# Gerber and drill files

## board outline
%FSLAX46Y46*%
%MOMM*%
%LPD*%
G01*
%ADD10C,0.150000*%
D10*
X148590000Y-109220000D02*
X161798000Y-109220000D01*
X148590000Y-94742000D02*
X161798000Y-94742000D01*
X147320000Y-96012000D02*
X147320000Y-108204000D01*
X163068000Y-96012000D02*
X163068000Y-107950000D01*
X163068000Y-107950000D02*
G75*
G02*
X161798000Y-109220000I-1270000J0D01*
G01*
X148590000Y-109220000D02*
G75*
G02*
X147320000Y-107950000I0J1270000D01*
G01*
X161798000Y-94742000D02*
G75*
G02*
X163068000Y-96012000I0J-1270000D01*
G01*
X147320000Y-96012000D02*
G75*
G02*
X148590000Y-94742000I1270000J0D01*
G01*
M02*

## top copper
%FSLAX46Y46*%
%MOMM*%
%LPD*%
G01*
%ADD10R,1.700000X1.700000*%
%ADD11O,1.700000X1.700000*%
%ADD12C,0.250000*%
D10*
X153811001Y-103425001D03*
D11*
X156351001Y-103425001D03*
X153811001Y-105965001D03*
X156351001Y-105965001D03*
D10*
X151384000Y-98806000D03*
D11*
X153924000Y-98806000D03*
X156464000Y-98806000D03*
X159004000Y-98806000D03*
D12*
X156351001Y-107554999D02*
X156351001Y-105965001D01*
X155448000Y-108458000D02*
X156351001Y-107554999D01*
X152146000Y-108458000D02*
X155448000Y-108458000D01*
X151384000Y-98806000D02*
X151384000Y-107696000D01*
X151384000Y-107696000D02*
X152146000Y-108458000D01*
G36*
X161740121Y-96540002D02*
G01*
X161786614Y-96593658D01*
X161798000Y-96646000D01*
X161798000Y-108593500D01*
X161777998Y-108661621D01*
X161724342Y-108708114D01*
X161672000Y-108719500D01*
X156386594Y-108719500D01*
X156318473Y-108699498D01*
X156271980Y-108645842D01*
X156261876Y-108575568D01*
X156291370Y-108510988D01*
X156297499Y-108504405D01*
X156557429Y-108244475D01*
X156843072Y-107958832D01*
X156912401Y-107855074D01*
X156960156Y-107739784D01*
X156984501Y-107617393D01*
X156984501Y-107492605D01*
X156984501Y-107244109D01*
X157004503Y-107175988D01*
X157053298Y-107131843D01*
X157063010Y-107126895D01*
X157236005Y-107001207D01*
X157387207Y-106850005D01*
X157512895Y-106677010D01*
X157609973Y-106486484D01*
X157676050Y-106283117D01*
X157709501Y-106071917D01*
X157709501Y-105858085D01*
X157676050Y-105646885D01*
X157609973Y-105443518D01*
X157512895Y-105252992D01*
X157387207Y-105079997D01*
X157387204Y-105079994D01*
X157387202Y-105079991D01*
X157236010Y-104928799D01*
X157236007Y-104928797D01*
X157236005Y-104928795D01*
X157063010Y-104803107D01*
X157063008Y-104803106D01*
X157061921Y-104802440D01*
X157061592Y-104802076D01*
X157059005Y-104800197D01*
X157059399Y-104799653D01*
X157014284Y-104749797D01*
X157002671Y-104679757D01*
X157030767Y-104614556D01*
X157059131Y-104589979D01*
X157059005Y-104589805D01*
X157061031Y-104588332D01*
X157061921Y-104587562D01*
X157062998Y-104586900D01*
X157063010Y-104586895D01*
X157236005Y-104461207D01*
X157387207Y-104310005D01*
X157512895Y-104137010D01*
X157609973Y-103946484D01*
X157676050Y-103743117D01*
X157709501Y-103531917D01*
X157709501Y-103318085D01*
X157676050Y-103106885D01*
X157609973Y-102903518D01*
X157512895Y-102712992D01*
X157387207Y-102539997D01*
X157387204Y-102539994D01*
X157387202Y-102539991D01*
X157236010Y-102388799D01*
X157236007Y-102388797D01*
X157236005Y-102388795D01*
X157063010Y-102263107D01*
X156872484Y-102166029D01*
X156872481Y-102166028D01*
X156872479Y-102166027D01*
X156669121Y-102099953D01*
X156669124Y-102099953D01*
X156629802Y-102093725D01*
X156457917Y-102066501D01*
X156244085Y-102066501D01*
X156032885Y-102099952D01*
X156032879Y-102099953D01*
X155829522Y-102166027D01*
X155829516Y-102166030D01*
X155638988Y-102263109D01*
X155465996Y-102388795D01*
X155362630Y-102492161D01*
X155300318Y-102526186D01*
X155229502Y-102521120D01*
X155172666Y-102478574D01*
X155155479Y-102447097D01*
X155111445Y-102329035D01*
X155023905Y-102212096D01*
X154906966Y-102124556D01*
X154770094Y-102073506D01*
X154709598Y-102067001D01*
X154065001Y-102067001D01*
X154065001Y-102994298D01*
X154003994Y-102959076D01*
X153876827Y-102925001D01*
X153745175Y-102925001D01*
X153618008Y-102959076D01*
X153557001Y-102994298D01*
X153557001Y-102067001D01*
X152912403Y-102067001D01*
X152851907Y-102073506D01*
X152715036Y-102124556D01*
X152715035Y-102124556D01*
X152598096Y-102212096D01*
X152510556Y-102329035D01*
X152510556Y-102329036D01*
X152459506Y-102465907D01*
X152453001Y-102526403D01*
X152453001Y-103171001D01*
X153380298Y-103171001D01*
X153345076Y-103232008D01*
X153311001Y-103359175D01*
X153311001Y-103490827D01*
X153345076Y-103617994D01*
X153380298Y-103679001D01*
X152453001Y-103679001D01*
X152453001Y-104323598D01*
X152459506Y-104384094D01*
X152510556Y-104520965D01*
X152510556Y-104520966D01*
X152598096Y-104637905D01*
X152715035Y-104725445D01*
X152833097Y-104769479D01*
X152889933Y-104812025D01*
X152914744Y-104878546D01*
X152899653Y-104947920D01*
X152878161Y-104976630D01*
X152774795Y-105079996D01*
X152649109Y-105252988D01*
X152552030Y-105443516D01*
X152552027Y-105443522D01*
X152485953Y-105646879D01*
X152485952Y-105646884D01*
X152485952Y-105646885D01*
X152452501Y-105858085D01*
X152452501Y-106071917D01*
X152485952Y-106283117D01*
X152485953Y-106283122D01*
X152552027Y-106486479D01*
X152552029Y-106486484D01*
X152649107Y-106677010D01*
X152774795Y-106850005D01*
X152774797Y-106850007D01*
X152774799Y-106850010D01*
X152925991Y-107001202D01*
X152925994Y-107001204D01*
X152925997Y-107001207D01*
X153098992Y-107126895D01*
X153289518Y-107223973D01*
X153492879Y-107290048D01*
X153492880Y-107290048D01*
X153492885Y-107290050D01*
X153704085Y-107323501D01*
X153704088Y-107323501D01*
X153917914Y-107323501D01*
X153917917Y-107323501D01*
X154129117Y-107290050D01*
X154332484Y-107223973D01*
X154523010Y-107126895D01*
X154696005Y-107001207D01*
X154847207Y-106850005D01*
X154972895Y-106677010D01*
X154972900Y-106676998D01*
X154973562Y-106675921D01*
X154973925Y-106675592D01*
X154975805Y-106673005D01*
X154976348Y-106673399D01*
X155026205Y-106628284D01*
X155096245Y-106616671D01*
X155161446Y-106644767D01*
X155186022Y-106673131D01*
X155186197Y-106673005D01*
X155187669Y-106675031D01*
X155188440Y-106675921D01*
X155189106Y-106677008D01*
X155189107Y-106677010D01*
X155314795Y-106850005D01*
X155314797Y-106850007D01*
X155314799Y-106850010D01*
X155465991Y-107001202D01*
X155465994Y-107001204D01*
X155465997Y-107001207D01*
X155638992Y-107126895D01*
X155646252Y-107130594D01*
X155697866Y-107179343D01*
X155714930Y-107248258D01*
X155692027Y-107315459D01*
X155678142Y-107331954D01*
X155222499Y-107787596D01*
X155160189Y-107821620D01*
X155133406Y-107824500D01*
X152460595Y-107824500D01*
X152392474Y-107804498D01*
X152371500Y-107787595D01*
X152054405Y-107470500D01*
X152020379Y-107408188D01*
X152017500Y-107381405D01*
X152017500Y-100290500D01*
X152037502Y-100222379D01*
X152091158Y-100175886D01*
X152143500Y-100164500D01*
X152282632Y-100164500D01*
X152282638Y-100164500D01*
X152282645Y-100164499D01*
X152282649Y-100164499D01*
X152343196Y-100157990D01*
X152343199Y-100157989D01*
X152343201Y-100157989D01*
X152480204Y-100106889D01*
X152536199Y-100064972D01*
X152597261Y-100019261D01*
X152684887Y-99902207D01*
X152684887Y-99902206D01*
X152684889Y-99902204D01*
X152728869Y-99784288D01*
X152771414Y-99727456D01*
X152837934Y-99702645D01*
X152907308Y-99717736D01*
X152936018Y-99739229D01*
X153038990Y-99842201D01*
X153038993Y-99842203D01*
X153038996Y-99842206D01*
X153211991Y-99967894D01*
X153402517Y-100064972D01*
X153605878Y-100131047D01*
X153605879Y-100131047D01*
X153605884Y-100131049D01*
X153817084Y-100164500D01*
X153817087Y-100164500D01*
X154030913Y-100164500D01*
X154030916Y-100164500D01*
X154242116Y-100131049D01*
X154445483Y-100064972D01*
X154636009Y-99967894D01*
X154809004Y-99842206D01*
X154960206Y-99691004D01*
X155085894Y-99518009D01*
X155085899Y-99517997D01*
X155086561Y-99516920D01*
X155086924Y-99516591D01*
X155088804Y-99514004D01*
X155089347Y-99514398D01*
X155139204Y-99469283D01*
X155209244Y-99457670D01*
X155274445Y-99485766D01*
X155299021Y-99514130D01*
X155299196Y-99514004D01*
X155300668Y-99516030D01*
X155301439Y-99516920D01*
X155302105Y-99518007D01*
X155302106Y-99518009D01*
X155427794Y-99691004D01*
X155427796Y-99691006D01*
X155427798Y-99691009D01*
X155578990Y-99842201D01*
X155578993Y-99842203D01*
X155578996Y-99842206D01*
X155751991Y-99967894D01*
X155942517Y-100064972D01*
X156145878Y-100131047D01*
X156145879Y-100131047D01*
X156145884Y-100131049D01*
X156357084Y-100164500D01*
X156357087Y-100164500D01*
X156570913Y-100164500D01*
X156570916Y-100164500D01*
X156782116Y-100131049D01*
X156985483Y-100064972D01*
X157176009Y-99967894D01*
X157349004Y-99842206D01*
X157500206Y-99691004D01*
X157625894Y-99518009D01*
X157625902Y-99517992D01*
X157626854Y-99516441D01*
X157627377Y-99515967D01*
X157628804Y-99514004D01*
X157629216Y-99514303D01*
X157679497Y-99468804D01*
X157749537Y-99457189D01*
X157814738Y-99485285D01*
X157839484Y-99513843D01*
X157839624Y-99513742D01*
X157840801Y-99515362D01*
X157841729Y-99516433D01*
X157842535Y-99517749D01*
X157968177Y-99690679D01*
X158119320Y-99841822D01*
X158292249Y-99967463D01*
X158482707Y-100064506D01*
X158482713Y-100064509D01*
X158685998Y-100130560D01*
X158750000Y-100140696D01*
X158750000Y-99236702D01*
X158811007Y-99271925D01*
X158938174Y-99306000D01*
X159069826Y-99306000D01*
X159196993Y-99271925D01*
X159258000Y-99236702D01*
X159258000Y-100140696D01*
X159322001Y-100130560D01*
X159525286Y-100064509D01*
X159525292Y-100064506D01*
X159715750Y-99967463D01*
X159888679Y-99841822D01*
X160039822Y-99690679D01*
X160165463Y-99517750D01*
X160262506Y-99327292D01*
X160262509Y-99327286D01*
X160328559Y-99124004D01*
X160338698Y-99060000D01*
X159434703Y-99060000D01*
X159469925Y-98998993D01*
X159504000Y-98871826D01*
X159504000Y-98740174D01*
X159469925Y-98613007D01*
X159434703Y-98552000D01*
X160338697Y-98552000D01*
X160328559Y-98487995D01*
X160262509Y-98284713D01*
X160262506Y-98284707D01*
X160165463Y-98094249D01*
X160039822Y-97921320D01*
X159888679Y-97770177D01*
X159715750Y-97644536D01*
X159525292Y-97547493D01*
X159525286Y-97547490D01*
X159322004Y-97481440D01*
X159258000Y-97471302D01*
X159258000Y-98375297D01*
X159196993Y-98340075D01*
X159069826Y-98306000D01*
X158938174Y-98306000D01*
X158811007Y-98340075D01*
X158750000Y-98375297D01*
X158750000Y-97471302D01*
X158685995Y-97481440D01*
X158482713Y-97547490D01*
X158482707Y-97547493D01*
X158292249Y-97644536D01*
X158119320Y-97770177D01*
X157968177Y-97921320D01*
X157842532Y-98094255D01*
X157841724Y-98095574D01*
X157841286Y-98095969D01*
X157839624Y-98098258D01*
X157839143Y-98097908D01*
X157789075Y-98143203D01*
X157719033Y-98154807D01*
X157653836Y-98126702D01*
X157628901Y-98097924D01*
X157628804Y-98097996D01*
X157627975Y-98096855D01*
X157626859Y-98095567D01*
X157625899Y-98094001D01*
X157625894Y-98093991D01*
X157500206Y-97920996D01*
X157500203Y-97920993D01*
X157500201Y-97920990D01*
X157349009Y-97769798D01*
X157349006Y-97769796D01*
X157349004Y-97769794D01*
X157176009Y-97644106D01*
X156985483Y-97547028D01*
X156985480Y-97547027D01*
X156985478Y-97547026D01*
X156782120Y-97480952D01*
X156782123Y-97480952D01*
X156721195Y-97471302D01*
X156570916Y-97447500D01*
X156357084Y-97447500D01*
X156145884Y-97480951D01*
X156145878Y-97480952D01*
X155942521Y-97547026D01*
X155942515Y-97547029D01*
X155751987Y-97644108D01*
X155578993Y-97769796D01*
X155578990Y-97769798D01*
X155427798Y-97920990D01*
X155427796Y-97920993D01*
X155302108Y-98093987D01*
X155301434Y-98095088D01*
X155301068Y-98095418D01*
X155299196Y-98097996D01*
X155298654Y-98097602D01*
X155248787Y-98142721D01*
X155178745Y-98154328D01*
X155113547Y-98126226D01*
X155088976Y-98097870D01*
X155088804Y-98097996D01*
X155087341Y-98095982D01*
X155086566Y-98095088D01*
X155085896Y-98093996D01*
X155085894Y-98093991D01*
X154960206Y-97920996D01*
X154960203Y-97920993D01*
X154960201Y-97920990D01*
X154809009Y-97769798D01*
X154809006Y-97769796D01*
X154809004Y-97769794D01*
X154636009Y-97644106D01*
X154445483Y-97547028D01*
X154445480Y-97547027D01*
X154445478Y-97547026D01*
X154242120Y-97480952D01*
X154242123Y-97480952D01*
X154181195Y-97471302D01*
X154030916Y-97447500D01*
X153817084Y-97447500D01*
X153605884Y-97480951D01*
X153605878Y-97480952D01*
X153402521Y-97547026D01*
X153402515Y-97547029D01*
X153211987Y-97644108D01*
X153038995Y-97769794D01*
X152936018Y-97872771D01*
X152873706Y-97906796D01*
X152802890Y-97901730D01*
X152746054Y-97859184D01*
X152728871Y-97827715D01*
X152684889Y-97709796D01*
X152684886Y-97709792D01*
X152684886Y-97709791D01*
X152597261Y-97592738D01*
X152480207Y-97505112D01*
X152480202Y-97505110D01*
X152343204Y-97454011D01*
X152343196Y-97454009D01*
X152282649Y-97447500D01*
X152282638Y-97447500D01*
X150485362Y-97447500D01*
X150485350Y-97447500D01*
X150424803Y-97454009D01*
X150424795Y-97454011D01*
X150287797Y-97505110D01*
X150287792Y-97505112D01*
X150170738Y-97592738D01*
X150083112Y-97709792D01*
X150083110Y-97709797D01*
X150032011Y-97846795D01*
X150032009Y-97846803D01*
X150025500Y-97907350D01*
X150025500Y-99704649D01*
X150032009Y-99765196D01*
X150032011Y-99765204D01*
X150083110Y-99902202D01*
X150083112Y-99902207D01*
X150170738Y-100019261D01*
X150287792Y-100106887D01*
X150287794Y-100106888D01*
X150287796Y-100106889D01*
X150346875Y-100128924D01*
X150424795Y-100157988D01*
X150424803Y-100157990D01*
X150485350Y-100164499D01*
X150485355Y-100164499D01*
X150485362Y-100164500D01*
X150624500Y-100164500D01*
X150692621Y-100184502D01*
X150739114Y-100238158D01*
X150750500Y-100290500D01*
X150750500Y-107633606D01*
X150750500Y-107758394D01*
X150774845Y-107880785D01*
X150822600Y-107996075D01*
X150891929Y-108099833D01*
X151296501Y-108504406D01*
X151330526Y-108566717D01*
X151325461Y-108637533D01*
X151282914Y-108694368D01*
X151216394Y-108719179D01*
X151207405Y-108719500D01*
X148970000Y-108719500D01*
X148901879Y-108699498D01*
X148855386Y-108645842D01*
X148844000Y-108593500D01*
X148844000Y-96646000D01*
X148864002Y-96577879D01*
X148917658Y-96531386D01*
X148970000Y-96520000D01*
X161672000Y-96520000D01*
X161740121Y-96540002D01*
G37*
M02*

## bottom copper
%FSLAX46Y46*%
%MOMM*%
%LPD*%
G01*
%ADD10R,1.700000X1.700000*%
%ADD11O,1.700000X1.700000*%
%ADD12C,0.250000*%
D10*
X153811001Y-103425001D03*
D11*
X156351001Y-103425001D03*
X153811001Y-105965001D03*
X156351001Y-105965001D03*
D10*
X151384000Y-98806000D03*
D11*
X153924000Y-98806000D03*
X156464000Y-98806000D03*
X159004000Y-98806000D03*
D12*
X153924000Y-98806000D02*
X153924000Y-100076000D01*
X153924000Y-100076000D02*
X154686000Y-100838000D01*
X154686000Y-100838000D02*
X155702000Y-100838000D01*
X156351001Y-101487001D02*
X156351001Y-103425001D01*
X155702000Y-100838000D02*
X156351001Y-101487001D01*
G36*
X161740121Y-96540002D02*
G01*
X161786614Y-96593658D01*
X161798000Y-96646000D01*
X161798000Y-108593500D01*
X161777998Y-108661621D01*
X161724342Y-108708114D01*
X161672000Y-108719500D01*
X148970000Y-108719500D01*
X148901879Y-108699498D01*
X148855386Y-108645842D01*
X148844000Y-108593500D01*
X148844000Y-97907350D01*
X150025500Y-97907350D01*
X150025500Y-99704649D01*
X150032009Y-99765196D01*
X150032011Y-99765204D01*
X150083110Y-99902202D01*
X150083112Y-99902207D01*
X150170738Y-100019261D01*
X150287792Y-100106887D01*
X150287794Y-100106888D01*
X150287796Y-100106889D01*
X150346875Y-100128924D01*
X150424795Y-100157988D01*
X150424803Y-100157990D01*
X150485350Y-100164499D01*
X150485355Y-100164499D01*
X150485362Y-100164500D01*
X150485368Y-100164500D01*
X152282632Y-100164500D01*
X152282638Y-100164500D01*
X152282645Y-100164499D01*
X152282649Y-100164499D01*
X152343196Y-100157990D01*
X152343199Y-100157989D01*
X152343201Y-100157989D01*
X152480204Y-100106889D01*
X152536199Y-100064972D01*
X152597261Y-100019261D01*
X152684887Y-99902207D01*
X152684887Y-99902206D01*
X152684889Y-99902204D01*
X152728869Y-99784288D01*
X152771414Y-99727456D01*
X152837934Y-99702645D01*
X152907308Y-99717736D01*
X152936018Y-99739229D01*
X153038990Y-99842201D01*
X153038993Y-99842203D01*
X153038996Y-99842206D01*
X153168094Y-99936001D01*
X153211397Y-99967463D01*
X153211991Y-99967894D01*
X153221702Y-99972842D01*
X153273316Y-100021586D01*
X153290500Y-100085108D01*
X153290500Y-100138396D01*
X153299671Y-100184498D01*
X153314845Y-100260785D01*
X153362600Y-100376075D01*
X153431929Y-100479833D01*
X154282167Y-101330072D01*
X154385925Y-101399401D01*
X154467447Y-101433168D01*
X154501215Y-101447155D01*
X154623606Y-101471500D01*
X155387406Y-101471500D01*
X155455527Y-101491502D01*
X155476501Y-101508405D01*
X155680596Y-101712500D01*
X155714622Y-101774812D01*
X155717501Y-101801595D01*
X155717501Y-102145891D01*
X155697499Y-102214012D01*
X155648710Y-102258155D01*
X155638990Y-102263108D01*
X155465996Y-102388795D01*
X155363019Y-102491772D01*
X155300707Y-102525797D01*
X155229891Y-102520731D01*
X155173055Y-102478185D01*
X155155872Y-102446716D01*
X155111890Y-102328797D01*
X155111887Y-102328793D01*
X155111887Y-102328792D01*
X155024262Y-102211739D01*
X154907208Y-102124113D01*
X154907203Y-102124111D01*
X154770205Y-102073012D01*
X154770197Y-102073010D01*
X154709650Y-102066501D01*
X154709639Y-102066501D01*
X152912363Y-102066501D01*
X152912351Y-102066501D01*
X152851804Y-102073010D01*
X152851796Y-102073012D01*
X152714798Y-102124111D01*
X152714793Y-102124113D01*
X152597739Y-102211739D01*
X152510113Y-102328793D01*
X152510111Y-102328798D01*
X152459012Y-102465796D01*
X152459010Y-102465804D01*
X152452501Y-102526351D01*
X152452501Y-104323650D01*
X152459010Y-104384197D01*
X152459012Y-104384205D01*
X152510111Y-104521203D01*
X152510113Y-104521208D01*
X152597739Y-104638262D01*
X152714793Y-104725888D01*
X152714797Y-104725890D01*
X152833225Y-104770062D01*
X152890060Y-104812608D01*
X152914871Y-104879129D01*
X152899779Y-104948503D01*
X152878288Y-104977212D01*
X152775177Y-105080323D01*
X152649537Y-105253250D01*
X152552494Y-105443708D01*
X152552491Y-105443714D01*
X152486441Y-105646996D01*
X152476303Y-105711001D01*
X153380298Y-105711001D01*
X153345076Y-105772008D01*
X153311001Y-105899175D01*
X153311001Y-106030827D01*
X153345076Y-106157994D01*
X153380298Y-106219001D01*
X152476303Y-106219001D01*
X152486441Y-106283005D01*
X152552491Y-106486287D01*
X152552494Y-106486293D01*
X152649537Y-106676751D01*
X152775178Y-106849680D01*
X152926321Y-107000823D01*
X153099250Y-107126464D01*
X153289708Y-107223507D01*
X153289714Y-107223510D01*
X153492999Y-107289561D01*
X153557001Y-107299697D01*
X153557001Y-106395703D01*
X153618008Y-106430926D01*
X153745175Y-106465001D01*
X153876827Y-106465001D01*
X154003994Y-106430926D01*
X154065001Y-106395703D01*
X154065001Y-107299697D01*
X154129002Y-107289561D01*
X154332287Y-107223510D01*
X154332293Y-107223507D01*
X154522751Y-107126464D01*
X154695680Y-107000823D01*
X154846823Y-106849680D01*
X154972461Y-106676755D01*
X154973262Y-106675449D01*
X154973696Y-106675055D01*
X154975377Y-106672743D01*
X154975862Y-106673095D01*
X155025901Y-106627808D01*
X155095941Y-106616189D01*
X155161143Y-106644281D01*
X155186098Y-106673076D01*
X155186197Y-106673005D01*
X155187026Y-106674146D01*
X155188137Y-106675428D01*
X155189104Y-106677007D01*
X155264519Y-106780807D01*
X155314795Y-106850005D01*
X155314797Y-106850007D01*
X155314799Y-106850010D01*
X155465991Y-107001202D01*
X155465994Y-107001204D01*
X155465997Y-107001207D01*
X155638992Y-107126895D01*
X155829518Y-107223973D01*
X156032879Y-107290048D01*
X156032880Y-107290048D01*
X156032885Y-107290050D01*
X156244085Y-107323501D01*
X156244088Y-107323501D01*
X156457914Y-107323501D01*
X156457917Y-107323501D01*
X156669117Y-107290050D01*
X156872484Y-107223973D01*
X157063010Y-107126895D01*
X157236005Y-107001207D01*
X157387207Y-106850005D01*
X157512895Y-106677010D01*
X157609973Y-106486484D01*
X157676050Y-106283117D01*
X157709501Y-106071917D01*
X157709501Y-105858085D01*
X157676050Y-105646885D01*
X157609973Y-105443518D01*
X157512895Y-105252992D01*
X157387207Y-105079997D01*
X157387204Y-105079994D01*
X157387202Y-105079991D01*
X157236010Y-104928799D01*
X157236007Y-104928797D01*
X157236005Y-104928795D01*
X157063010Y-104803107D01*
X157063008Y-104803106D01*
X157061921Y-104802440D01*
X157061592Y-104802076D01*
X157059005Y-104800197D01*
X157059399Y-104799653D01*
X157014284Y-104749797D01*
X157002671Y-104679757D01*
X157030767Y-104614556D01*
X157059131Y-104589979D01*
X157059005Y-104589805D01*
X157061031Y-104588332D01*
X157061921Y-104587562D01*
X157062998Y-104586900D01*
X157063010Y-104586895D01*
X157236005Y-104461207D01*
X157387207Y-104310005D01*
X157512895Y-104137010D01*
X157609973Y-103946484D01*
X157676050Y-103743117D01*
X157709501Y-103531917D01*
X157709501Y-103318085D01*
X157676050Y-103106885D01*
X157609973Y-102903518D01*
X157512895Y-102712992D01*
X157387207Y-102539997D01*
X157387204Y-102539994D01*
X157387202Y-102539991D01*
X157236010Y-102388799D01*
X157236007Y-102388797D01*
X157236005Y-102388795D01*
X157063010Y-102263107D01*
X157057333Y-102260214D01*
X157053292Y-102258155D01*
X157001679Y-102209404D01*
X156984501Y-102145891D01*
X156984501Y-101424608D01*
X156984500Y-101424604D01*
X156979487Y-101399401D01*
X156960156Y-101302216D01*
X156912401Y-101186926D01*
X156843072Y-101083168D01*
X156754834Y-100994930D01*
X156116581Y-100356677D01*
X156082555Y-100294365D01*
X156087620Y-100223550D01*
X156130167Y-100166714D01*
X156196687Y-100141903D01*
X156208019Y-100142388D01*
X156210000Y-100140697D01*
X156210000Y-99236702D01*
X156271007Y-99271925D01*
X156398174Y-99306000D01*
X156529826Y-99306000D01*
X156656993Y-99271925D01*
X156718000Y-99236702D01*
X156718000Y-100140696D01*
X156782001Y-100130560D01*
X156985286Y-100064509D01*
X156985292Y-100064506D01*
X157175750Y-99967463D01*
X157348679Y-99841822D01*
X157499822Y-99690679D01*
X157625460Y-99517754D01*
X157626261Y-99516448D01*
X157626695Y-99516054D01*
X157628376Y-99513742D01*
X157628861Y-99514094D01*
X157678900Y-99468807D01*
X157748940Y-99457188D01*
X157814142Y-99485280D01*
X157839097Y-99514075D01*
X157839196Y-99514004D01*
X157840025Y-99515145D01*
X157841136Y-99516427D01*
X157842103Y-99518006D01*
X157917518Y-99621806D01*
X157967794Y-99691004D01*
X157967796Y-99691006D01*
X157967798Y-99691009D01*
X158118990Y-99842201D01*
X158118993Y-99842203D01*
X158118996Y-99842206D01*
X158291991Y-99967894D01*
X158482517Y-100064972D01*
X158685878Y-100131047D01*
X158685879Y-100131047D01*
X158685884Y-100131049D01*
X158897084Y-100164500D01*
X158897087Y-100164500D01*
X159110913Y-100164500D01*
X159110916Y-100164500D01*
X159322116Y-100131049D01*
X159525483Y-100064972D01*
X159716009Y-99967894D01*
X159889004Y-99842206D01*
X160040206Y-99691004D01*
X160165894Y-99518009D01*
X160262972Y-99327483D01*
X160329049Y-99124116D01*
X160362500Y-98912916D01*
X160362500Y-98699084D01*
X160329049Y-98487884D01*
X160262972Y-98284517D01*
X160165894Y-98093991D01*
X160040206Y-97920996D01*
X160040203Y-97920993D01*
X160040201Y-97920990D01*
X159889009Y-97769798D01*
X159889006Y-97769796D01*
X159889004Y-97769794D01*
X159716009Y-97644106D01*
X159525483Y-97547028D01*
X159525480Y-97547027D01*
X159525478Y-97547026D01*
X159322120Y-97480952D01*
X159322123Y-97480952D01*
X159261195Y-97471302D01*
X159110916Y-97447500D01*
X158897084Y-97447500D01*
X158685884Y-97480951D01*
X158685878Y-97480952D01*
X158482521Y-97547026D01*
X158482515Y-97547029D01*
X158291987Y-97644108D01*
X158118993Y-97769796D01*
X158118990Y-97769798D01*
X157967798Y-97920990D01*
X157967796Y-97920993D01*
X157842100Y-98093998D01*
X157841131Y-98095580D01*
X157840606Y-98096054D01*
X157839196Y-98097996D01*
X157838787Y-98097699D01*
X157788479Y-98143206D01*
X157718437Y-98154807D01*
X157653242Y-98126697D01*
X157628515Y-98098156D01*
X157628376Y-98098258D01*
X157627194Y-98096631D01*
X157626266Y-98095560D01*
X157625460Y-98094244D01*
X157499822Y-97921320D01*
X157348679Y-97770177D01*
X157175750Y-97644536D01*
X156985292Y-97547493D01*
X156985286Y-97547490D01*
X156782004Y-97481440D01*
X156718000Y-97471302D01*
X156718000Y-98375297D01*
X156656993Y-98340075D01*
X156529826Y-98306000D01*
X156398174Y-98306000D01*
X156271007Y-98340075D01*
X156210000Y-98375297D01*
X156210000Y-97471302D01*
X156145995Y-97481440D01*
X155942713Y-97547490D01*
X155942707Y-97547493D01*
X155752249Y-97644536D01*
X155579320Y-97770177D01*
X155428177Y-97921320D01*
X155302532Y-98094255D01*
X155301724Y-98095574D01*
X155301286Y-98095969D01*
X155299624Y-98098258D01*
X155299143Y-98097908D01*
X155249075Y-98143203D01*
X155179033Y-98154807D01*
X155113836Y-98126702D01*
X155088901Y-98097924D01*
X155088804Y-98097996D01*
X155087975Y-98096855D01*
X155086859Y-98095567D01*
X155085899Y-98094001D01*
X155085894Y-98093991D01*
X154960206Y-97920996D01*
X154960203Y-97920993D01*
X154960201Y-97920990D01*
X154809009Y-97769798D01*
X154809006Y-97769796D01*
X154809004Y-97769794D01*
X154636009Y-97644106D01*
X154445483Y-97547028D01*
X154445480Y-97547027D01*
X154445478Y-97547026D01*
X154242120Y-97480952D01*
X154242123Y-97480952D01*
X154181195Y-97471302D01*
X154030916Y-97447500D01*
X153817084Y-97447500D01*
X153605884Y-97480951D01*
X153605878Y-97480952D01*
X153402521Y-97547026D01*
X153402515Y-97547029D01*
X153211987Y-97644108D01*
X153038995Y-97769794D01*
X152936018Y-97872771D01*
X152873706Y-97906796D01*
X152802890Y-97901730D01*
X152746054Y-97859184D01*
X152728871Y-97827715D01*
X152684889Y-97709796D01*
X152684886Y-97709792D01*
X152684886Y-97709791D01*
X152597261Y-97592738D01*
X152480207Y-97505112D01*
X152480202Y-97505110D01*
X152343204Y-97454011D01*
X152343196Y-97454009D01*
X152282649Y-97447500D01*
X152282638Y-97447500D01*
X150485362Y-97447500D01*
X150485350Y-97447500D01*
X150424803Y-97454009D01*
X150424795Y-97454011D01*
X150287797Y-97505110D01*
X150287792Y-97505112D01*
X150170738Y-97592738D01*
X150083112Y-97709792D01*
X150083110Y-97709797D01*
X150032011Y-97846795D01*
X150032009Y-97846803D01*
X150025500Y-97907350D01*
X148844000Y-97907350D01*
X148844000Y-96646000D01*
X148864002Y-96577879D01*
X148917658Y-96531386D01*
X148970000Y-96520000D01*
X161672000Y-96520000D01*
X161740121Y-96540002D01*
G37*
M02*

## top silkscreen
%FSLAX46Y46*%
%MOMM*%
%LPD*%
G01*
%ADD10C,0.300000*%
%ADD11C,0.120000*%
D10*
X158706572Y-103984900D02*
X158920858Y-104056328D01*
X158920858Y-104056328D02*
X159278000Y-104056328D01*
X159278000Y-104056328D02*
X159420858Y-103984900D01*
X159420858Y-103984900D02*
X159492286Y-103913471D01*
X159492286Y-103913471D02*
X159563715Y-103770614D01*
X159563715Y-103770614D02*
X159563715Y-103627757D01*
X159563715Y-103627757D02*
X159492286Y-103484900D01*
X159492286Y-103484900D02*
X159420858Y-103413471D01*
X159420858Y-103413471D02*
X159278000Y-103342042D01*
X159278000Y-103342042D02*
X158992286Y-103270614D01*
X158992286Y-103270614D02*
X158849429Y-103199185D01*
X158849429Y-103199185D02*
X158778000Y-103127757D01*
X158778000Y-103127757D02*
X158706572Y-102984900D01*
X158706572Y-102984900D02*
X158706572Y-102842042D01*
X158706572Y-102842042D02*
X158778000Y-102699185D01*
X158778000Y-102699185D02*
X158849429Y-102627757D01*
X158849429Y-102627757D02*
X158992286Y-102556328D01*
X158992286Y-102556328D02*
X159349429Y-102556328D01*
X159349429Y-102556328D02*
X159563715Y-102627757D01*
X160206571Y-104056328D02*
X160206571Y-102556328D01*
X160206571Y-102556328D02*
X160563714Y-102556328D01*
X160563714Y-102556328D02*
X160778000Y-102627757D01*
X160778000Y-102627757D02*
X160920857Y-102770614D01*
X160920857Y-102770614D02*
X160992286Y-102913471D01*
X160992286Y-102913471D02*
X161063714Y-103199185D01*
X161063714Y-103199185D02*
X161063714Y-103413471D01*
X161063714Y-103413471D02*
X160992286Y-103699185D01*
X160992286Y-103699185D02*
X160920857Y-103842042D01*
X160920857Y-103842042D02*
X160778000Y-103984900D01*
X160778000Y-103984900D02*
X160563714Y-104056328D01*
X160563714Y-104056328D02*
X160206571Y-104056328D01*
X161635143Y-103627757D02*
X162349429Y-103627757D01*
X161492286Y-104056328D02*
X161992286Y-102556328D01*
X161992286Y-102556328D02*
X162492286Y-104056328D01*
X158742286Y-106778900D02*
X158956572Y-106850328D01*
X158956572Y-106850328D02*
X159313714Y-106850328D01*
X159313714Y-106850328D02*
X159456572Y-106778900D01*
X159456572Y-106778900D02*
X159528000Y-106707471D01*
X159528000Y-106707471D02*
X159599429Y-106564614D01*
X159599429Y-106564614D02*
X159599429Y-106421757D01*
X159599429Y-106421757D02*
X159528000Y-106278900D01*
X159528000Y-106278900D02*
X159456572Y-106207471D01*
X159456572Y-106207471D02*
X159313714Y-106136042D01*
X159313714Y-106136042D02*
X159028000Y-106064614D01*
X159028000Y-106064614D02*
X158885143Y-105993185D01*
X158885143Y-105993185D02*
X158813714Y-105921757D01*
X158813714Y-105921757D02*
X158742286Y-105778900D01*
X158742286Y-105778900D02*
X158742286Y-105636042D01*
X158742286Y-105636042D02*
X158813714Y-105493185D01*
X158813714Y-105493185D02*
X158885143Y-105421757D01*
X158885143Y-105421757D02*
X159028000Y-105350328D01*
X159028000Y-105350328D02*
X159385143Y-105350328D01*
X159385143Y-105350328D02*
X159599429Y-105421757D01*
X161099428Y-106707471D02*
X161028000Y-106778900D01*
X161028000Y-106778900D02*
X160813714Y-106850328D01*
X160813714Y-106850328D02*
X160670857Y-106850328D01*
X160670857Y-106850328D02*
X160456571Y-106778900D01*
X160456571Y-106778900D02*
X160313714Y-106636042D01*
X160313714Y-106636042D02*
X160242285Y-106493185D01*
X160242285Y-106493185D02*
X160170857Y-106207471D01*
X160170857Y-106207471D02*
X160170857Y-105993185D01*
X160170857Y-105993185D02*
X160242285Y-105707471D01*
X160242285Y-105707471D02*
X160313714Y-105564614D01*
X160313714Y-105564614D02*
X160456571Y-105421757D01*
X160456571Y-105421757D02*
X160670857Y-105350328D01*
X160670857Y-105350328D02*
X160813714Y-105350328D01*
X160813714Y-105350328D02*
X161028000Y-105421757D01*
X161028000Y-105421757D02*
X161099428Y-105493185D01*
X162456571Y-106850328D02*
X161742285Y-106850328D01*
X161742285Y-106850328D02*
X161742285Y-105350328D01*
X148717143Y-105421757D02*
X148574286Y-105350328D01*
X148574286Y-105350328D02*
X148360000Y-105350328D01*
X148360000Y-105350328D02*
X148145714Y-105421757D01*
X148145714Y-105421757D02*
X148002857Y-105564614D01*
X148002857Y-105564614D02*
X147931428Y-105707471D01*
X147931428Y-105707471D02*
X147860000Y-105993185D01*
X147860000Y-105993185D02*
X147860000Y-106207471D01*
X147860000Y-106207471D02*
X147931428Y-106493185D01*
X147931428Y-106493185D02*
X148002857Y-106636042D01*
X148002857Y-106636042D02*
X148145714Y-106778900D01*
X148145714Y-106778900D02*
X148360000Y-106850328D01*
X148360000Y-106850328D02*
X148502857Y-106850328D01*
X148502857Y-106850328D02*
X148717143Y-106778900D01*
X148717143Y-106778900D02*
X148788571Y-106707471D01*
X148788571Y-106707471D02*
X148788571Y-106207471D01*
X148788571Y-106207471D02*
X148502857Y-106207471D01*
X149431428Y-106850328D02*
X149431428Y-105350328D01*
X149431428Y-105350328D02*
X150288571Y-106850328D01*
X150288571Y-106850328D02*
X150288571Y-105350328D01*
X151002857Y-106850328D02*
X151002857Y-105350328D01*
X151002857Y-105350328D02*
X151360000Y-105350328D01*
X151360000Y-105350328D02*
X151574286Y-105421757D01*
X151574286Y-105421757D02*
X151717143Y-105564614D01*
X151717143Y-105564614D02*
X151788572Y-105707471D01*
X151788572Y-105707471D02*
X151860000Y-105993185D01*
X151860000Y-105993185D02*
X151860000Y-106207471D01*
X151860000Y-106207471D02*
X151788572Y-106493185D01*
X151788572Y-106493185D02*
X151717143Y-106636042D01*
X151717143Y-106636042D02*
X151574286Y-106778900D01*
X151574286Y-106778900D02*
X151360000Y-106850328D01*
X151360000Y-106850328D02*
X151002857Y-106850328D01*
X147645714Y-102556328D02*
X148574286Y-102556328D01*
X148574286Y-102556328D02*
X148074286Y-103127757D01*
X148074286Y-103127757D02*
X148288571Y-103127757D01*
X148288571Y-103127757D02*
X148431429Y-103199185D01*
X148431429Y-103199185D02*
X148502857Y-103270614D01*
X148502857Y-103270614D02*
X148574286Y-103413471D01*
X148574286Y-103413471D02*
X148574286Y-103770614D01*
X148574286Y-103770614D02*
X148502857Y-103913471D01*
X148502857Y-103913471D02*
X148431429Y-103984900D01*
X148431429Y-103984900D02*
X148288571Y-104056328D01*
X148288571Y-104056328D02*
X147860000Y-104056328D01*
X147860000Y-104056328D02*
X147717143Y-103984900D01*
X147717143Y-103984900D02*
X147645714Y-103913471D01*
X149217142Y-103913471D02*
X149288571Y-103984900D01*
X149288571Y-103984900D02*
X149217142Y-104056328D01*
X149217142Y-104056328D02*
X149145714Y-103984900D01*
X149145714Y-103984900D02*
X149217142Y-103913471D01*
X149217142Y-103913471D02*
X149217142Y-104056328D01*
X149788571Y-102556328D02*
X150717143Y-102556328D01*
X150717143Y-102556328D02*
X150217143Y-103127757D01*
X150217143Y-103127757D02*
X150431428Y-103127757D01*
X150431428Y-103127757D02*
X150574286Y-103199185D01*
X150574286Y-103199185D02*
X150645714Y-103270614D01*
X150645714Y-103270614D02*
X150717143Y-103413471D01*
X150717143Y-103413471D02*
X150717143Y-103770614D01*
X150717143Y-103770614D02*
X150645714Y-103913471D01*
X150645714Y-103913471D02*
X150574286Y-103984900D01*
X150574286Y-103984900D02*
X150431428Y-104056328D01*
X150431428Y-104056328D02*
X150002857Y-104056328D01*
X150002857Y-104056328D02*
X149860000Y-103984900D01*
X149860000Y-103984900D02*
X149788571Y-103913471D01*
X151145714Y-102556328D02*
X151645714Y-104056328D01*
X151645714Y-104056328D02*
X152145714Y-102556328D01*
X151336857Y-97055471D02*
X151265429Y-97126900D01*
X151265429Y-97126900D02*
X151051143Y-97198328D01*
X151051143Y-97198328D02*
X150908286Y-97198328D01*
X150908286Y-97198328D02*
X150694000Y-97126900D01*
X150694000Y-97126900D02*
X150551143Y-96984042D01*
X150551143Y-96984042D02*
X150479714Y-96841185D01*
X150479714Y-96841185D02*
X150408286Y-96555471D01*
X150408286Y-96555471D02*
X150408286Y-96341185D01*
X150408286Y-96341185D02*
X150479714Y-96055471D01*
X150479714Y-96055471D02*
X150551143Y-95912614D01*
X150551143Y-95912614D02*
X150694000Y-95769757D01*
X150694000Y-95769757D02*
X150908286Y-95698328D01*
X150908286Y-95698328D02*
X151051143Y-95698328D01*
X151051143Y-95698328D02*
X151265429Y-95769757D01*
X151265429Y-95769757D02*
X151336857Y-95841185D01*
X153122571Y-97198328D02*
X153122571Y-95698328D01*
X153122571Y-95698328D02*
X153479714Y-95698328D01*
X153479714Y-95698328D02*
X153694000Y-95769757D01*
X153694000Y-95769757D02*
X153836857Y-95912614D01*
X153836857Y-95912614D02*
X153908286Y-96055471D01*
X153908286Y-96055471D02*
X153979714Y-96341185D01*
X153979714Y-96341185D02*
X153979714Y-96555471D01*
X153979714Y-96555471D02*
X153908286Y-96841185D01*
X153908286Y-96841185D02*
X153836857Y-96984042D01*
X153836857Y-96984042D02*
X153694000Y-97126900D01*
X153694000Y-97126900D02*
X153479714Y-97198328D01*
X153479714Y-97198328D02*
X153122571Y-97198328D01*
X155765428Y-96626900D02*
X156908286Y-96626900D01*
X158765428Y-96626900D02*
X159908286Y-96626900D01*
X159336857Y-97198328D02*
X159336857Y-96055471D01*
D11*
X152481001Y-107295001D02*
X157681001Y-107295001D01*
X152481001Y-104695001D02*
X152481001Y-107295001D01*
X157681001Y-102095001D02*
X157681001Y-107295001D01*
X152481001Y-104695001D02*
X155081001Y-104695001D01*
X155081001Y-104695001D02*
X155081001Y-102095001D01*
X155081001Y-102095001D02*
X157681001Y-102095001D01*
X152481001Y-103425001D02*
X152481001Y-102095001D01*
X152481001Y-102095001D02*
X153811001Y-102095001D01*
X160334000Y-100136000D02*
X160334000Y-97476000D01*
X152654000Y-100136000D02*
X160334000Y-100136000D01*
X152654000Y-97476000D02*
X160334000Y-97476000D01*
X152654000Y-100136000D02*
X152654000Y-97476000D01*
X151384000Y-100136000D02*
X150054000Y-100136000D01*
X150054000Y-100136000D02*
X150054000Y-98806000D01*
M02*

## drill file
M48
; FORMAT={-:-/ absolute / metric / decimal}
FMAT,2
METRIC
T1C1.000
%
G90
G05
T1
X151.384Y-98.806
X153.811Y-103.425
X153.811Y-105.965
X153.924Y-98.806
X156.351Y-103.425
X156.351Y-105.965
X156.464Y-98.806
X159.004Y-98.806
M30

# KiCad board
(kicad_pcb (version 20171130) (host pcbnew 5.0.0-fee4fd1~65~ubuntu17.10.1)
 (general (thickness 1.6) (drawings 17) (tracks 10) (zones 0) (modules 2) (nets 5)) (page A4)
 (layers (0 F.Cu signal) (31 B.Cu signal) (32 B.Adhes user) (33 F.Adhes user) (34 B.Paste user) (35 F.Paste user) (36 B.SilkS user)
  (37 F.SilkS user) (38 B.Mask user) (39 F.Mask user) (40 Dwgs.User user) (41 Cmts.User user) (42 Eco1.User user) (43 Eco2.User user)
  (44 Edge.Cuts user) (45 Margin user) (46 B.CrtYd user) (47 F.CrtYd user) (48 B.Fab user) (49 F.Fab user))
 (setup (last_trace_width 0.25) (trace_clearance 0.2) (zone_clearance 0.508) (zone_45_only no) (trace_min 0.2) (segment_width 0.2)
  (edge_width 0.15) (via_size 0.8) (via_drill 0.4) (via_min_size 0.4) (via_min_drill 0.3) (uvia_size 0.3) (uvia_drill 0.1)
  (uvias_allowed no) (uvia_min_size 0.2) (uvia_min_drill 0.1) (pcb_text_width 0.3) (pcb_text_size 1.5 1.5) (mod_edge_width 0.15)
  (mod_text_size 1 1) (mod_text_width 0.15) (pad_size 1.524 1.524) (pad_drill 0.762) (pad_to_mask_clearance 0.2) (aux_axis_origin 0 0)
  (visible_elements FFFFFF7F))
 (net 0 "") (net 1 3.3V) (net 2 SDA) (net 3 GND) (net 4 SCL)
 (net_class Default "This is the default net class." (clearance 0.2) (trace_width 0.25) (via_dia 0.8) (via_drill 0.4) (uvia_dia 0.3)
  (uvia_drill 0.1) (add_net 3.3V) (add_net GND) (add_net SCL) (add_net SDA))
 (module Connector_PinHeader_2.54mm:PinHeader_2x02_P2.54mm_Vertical (layer F.Cu) (at 153.811001 103.425001)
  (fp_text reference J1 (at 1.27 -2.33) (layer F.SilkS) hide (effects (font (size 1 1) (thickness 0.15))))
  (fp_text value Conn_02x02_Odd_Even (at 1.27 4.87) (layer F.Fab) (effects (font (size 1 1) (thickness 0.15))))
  (fp_line (start -1.33 3.87) (end 3.87 3.87) (layer F.SilkS) (width 0.12))
  (fp_line (start -1.33 1.27) (end -1.33 3.87) (layer F.SilkS) (width 0.12))
  (fp_line (start 3.87 -1.33) (end 3.87 3.87) (layer F.SilkS) (width 0.12))
  (fp_line (start -1.33 1.27) (end 1.27 1.27) (layer F.SilkS) (width 0.12))
  (fp_line (start 1.27 1.27) (end 1.27 -1.33) (layer F.SilkS) (width 0.12))
  (fp_line (start 1.27 -1.33) (end 3.87 -1.33) (layer F.SilkS) (width 0.12))
  (fp_line (start -1.33 0) (end -1.33 -1.33) (layer F.SilkS) (width 0.12))
  (fp_line (start -1.33 -1.33) (end 0 -1.33) (layer F.SilkS) (width 0.12))
  (pad 1 thru_hole rect (at 0 0) (size 1.7 1.7) (drill 1) (layers *.Cu *.Mask) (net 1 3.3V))
  (pad 2 thru_hole oval (at 2.54 0) (size 1.7 1.7) (drill 1) (layers *.Cu *.Mask) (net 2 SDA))
  (pad 3 thru_hole oval (at 0 2.54) (size 1.7 1.7) (drill 1) (layers *.Cu *.Mask) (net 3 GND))
  (pad 4 thru_hole oval (at 2.54 2.54) (size 1.7 1.7) (drill 1) (layers *.Cu *.Mask) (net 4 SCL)))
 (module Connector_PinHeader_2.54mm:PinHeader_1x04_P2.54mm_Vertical (layer F.Cu) (at 151.384 98.806 90)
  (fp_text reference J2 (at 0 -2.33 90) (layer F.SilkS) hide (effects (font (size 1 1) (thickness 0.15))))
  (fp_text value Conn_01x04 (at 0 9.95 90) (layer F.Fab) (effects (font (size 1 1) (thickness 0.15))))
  (fp_line (start -1.33 8.95) (end 1.33 8.95) (layer F.SilkS) (width 0.12))
  (fp_line (start -1.33 1.27) (end -1.33 8.95) (layer F.SilkS) (width 0.12))
  (fp_line (start 1.33 1.27) (end 1.33 8.95) (layer F.SilkS) (width 0.12))
  (fp_line (start -1.33 1.27) (end 1.33 1.27) (layer F.SilkS) (width 0.12))
  (fp_line (start -1.33 0) (end -1.33 -1.33) (layer F.SilkS) (width 0.12))
  (fp_line (start -1.33 -1.33) (end 0 -1.33) (layer F.SilkS) (width 0.12))
  (pad 1 thru_hole rect (at 0 0 90) (size 1.7 1.7) (drill 1) (layers *.Cu *.Mask) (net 4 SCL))
  (pad 2 thru_hole oval (at 0 2.54 90) (size 1.7 1.7) (drill 1) (layers *.Cu *.Mask) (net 2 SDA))
  (pad 3 thru_hole oval (at 0 5.08 90) (size 1.7 1.7) (drill 1) (layers *.Cu *.Mask) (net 3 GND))
  (pad 4 thru_hole oval (at 0 7.62 90) (size 1.7 1.7) (drill 1) (layers *.Cu *.Mask) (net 1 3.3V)))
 (gr_line (start 148.59 109.22) (end 161.798 109.22) (layer Edge.Cuts) (width 0.15))
 (gr_line (start 148.59 94.742) (end 161.798 94.742) (layer Edge.Cuts) (width 0.15))
 (gr_line (start 147.32 96.012) (end 147.32 108.204) (layer Edge.Cuts) (width 0.15))
 (gr_line (start 163.068 96.012) (end 163.068 107.95) (layer Edge.Cuts) (width 0.15))
 (gr_arc (start 161.798 107.95) (end 161.798 109.22) (angle -90) (layer Edge.Cuts) (width 0.15))
 (gr_arc (start 148.59 107.95) (end 147.32 107.95) (angle -90) (layer Edge.Cuts) (width 0.15))
 (gr_arc (start 161.798 96.012) (end 163.068 96.012) (angle -90) (layer Edge.Cuts) (width 0.15))
 (gr_arc (start 148.59 96.012) (end 148.59 94.742) (angle -90) (layer Edge.Cuts) (width 0.15))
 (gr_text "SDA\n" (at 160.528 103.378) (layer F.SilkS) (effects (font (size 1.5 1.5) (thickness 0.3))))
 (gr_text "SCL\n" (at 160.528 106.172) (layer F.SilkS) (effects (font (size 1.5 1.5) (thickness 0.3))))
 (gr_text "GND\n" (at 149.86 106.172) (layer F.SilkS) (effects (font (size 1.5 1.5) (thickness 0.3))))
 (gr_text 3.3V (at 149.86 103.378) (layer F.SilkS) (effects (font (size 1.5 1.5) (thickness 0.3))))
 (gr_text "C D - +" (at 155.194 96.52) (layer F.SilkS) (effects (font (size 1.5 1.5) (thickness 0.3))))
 (segment (start 153.924 98.806) (end 153.924 100.076) (width 0.25) (layer B.Cu) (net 2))
 (segment (start 153.924 100.076) (end 154.686 100.838) (width 0.25) (layer B.Cu) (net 2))
 (segment (start 154.686 100.838) (end 155.702 100.838) (width 0.25) (layer B.Cu) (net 2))
 (segment (start 156.351001 101.487001) (end 156.351001 103.425001) (width 0.25) (layer B.Cu) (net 2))
 (segment (start 155.702 100.838) (end 156.351001 101.487001) (width 0.25) (layer B.Cu) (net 2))
 (segment (start 156.351001 107.554999) (end 156.351001 105.965001) (width 0.25) (layer F.Cu) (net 4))
 (segment (start 155.448 108.458) (end 156.351001 107.554999) (width 0.25) (layer F.Cu) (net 4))
 (segment (start 152.146 108.458) (end 155.448 108.458) (width 0.25) (layer F.Cu) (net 4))
 (segment (start 151.384 98.806) (end 151.384 107.696) (width 0.25) (layer F.Cu) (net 4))
 (segment (start 151.384 107.696) (end 152.146 108.458) (width 0.25) (layer F.Cu) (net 4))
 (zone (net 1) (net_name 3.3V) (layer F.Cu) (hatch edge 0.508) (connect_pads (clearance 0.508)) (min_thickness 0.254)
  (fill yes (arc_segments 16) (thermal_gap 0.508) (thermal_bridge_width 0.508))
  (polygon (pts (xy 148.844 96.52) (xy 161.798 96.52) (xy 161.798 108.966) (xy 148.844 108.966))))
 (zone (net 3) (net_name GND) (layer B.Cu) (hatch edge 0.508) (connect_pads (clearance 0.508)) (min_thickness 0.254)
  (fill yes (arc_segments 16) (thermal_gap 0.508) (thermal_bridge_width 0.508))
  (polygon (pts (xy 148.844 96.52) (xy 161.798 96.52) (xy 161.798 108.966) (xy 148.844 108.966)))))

